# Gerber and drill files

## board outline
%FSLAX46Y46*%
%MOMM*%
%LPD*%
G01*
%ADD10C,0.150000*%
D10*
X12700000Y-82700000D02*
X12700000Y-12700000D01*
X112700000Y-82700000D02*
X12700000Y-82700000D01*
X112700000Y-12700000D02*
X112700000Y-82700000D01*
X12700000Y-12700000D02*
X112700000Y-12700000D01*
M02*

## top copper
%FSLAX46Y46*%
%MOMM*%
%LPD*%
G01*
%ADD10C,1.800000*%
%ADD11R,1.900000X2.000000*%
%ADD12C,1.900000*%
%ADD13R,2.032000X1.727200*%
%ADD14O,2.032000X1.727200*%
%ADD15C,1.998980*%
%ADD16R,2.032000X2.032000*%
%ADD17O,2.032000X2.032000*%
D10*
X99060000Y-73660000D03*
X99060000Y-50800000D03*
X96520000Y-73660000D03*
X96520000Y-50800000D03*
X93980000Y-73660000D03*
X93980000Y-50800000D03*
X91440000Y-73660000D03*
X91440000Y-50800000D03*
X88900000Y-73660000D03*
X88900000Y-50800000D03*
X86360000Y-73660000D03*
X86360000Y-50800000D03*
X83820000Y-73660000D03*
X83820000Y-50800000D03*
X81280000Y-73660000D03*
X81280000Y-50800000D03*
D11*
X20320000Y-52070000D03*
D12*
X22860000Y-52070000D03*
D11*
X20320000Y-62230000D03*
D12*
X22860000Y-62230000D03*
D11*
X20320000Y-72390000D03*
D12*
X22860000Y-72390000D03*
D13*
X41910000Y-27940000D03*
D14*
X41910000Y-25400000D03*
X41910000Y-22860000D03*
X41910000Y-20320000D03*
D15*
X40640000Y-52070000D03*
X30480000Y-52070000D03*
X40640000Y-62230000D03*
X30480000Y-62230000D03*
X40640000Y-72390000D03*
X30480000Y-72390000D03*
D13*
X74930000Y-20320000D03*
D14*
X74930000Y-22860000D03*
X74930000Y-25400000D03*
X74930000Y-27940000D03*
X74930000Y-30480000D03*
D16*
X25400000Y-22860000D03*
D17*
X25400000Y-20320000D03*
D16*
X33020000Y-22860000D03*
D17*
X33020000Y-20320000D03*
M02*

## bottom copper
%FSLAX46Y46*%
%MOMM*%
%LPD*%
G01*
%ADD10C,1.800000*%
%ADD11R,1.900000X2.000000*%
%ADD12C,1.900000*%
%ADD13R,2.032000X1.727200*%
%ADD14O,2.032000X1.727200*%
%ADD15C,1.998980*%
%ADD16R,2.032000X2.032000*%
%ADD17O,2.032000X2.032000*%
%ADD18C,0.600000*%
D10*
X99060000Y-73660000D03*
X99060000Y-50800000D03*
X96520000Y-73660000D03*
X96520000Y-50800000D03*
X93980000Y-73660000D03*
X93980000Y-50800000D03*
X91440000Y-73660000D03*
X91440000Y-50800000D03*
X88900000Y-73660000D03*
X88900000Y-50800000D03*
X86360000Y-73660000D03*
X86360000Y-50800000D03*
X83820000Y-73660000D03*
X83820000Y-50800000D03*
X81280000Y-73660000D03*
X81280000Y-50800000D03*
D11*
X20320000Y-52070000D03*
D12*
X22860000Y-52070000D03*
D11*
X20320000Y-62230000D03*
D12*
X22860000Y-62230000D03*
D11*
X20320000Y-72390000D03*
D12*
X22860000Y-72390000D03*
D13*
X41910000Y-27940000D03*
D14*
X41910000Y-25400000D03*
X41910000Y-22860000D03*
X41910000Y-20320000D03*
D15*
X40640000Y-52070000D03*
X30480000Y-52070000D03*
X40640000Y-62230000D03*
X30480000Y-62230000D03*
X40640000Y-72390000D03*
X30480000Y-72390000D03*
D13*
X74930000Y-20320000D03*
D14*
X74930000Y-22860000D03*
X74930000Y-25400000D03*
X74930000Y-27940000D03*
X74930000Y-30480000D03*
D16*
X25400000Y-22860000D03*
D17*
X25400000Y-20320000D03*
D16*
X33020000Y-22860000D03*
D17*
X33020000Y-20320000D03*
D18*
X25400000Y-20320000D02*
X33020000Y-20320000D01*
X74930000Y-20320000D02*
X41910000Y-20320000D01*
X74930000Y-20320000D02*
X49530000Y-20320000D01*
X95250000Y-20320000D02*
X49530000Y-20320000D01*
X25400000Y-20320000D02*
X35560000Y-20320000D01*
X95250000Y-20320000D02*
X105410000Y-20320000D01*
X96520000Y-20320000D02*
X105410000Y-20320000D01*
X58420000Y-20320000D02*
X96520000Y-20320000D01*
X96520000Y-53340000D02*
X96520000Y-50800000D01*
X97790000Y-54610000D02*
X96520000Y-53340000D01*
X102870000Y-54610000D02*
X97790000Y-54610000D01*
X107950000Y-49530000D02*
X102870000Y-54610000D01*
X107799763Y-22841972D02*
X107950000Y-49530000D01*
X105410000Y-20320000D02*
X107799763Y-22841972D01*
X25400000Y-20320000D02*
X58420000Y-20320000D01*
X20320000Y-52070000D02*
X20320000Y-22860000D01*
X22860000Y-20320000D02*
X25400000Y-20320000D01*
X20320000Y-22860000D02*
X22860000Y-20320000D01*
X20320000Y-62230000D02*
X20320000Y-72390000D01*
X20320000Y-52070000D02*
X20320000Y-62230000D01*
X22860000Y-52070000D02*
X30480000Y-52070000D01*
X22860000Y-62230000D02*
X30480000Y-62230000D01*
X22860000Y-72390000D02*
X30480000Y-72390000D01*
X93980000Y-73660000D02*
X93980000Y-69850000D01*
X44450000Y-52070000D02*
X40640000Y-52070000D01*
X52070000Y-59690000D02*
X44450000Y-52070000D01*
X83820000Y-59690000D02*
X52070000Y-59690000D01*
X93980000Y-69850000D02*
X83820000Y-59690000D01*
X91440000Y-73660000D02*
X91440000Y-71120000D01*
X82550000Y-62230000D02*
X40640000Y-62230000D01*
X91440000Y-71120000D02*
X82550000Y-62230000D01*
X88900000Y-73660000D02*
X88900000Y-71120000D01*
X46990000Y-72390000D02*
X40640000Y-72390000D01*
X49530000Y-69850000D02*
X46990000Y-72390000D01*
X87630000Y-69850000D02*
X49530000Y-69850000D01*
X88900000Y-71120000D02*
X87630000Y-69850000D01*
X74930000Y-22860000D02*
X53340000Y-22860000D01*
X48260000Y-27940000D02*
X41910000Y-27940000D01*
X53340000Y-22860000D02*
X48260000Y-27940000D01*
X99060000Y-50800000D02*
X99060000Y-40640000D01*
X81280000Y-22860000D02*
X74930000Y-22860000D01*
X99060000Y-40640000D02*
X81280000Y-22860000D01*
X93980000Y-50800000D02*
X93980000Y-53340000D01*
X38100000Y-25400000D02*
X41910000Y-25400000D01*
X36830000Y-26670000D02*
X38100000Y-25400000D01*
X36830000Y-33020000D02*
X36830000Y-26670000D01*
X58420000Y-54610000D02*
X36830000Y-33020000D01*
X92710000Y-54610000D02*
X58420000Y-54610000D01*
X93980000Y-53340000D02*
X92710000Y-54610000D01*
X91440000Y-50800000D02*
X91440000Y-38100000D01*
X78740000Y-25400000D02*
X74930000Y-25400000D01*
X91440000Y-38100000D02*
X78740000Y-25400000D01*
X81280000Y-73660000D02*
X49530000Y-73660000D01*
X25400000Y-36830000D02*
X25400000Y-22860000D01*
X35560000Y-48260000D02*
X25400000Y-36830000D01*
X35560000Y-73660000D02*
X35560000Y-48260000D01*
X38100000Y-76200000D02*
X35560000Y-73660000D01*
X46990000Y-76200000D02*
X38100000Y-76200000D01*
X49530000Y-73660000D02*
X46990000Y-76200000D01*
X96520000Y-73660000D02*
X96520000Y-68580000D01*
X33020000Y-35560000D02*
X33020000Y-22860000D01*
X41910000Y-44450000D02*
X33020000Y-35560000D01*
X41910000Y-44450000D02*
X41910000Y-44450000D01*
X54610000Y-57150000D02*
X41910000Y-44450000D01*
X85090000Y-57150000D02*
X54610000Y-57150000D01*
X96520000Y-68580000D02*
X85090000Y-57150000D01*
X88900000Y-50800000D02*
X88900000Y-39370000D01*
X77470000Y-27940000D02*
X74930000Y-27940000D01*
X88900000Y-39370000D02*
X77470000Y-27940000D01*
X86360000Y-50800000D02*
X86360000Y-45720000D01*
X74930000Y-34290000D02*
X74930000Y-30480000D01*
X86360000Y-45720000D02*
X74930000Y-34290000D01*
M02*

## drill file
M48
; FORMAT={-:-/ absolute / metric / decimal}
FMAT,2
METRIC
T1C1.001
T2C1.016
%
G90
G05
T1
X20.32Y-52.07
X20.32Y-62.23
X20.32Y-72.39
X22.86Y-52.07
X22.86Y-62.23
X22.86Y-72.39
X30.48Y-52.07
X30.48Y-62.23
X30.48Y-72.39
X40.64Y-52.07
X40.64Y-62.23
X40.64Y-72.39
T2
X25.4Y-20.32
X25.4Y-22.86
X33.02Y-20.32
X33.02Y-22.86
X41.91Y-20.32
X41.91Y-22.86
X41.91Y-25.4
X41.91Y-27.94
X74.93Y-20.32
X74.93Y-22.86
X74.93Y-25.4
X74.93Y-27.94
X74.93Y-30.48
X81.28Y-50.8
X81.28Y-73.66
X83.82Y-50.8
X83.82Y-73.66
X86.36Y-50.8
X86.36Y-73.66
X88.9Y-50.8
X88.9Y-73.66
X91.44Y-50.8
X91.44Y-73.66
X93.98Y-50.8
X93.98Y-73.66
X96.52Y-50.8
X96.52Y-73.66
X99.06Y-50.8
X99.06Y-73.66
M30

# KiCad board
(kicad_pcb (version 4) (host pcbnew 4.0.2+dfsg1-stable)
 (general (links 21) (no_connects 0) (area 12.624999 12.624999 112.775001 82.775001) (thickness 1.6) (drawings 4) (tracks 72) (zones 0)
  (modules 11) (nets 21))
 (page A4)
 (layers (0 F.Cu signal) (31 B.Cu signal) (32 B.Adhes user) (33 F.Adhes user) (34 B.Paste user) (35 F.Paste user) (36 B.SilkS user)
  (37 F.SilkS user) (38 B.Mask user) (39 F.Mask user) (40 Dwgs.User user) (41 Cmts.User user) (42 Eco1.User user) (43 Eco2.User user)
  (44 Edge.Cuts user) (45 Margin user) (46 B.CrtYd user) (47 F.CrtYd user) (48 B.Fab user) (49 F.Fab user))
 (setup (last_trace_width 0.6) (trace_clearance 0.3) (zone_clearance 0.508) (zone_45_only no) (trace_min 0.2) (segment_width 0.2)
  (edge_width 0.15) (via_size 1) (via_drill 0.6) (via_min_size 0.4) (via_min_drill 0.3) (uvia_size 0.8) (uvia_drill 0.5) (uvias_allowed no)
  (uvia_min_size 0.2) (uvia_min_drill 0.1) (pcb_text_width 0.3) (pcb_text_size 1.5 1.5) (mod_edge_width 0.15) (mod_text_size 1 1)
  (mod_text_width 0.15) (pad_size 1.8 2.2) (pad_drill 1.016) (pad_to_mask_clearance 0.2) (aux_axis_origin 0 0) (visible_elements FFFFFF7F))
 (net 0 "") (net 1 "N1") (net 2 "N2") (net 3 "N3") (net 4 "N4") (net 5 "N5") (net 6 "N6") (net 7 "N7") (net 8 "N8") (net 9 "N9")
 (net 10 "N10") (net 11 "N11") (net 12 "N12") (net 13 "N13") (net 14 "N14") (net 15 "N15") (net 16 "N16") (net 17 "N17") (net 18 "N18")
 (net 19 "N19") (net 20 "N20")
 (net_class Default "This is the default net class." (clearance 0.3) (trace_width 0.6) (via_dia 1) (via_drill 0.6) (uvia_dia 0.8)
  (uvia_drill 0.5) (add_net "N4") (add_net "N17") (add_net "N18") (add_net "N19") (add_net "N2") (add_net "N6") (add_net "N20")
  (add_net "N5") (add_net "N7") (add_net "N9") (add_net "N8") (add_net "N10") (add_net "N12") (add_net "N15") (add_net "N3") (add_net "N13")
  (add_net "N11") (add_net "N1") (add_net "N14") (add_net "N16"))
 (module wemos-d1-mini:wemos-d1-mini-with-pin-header (layer F.Cu) (at 90.17 62.23 180)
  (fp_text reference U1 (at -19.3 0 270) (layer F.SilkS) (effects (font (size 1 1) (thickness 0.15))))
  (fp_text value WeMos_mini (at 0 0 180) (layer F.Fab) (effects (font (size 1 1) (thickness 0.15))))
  (pad 16 thru_hole circle (at -8.89 -11.43 180) (size 1.8 1.8) (drill 1.016) (layers *.Cu *.Mask) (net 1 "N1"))
  (pad 1 thru_hole circle (at -8.89 11.43 180) (size 1.8 1.8) (drill 1.016) (layers *.Cu *.Mask) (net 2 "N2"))
  (pad 15 thru_hole circle (at -6.35 -11.43 180) (size 1.8 1.8) (drill 1.016) (layers *.Cu *.Mask) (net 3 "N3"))
  (pad 2 thru_hole circle (at -6.35 11.43 180) (size 1.8 1.8) (drill 1.016) (layers *.Cu *.Mask) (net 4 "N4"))
  (pad 14 thru_hole circle (at -3.81 -11.43 180) (size 1.8 1.8) (drill 1.016) (layers *.Cu *.Mask) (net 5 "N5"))
  (pad 3 thru_hole circle (at -3.81 11.43 180) (size 1.8 1.8) (drill 1.016) (layers *.Cu *.Mask) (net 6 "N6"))
  (pad 13 thru_hole circle (at -1.27 -11.43 180) (size 1.8 1.8) (drill 1.016) (layers *.Cu *.Mask) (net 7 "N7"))
  (pad 4 thru_hole circle (at -1.27 11.43 180) (size 1.8 1.8) (drill 1.016) (layers *.Cu *.Mask) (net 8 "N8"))
  (pad 12 thru_hole circle (at 1.27 -11.43 180) (size 1.8 1.8) (drill 1.016) (layers *.Cu *.Mask) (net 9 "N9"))
  (pad 5 thru_hole circle (at 1.27 11.43 180) (size 1.8 1.8) (drill 1.016) (layers *.Cu *.Mask) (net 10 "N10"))
  (pad 11 thru_hole circle (at 3.81 -11.43 180) (size 1.8 1.8) (drill 1.016) (layers *.Cu *.Mask) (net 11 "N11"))
  (pad 6 thru_hole circle (at 3.81 11.43 180) (size 1.8 1.8) (drill 1.016) (layers *.Cu *.Mask) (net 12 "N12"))
  (pad 10 thru_hole circle (at 6.35 -11.43 180) (size 1.8 1.8) (drill 1.016) (layers *.Cu *.Mask) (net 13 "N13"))
  (pad 7 thru_hole circle (at 6.35 11.43 180) (size 1.8 1.8) (drill 1.016) (layers *.Cu *.Mask) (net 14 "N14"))
  (pad 9 thru_hole circle (at 8.89 -11.43 180) (size 1.8 1.8) (drill 1.016) (layers *.Cu *.Mask) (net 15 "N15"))
  (pad 8 thru_hole circle (at 8.89 11.43 180) (size 1.8 1.8) (drill 1.016) (layers *.Cu *.Mask) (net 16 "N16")))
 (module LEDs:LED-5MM (layer F.Cu) (at 20.32 52.07)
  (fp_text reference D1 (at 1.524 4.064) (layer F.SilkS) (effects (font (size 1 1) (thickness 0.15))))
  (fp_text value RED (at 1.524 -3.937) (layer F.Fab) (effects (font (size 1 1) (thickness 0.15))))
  (pad 1 thru_hole rect (at 0 0 90) (size 2 1.9) (drill 1.00076) (layers *.Cu *.Mask F.SilkS) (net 4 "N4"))
  (pad 2 thru_hole circle (at 2.54 0) (size 1.9 1.9) (drill 1.00076) (layers *.Cu *.Mask F.SilkS) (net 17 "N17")))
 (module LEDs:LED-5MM (layer F.Cu) (at 20.32 62.23)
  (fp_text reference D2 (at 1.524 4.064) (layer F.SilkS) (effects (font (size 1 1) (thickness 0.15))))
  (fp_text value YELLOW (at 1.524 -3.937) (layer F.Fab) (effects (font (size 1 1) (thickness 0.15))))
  (pad 1 thru_hole rect (at 0 0 90) (size 2 1.9) (drill 1.00076) (layers *.Cu *.Mask F.SilkS) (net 4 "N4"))
  (pad 2 thru_hole circle (at 2.54 0) (size 1.9 1.9) (drill 1.00076) (layers *.Cu *.Mask F.SilkS) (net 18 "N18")))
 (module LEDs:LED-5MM (layer F.Cu) (at 20.32 72.39)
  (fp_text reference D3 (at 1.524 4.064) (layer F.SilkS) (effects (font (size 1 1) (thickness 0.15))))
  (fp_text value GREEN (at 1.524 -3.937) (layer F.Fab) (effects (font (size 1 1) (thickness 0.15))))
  (pad 1 thru_hole rect (at 0 0 90) (size 2 1.9) (drill 1.00076) (layers *.Cu *.Mask F.SilkS) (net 4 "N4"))
  (pad 2 thru_hole circle (at 2.54 0) (size 1.9 1.9) (drill 1.00076) (layers *.Cu *.Mask F.SilkS) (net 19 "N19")))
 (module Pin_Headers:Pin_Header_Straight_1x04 (layer F.Cu) (at 41.91 27.94 180)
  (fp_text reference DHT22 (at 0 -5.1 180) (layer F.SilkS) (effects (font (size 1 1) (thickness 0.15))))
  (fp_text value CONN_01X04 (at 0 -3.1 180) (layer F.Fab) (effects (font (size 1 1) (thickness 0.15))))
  (pad 1 thru_hole rect (at 0 0 180) (size 2.032 1.7272) (drill 1.016) (layers *.Cu *.Mask F.SilkS) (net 2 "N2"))
  (pad 2 thru_hole oval (at 0 2.54 180) (size 2.032 1.7272) (drill 1.016) (layers *.Cu *.Mask F.SilkS) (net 6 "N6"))
  (pad 3 thru_hole oval (at 0 5.08 180) (size 2.032 1.7272) (drill 1.016) (layers *.Cu *.Mask F.SilkS) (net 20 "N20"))
  (pad 4 thru_hole oval (at 0 7.62 180) (size 2.032 1.7272) (drill 1.016) (layers *.Cu *.Mask F.SilkS) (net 4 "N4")))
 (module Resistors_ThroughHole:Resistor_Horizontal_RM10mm (layer F.Cu) (at 40.64 52.07 180)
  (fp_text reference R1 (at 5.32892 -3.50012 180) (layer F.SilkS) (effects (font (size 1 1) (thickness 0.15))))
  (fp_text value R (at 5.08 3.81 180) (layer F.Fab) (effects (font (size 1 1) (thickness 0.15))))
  (pad 1 thru_hole circle (at 0 0 180) (size 1.99898 1.99898) (drill 1.00076) (layers *.Cu *.SilkS *.Mask) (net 5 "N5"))
  (pad 2 thru_hole circle (at 10.16 0 180) (size 1.99898 1.99898) (drill 1.00076) (layers *.Cu *.SilkS *.Mask) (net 17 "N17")))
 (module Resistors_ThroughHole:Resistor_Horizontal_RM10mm (layer F.Cu) (at 40.64 62.23 180)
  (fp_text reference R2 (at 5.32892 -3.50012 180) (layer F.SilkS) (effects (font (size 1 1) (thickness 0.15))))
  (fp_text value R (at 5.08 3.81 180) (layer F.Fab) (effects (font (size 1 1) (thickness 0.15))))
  (pad 1 thru_hole circle (at 0 0 180) (size 1.99898 1.99898) (drill 1.00076) (layers *.Cu *.SilkS *.Mask) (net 7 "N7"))
  (pad 2 thru_hole circle (at 10.16 0 180) (size 1.99898 1.99898) (drill 1.00076) (layers *.Cu *.SilkS *.Mask) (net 18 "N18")))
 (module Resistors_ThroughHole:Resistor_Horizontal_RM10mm (layer F.Cu) (at 40.64 72.39 180)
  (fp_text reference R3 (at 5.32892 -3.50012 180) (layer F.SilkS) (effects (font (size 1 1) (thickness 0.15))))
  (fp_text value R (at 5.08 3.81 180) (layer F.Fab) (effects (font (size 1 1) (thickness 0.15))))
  (pad 1 thru_hole circle (at 0 0 180) (size 1.99898 1.99898) (drill 1.00076) (layers *.Cu *.SilkS *.Mask) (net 9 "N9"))
  (pad 2 thru_hole circle (at 10.16 0 180) (size 1.99898 1.99898) (drill 1.00076) (layers *.Cu *.SilkS *.Mask) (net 19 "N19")))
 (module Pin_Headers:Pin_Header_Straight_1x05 (layer F.Cu) (at 74.93 20.32)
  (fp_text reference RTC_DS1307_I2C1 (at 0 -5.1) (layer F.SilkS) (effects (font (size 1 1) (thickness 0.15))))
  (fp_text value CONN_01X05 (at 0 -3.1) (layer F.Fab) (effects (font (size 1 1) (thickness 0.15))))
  (pad 1 thru_hole rect (at 0 0) (size 2.032 1.7272) (drill 1.016) (layers *.Cu *.Mask F.SilkS) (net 4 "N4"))
  (pad 2 thru_hole oval (at 0 2.54) (size 2.032 1.7272) (drill 1.016) (layers *.Cu *.Mask F.SilkS) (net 2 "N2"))
  (pad 3 thru_hole oval (at 0 5.08) (size 2.032 1.7272) (drill 1.016) (layers *.Cu *.Mask F.SilkS) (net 8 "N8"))
  (pad 4 thru_hole oval (at 0 7.62) (size 2.032 1.7272) (drill 1.016) (layers *.Cu *.Mask F.SilkS) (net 10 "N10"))
  (pad 5 thru_hole oval (at 0 10.16) (size 2.032 1.7272) (drill 1.016) (layers *.Cu *.Mask F.SilkS) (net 12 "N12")))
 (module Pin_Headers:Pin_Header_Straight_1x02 (layer F.Cu) (at 25.4 22.86 180)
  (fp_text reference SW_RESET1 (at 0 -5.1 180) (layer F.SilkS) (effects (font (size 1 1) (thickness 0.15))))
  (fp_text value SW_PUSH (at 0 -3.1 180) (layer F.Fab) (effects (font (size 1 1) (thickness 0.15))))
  (pad 1 thru_hole rect (at 0 0 180) (size 2.032 2.032) (drill 1.016) (layers *.Cu *.Mask F.SilkS) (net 15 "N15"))
  (pad 2 thru_hole oval (at 0 2.54 180) (size 2.032 2.032) (drill 1.016) (layers *.Cu *.Mask F.SilkS) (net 4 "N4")))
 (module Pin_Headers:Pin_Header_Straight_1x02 (layer F.Cu) (at 33.02 22.86 180)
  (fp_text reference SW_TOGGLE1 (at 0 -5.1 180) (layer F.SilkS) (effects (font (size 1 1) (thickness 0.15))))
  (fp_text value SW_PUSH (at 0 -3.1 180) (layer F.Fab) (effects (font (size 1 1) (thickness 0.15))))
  (pad 1 thru_hole rect (at 0 0 180) (size 2.032 2.032) (drill 1.016) (layers *.Cu *.Mask F.SilkS) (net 3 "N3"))
  (pad 2 thru_hole oval (at 0 2.54 180) (size 2.032 2.032) (drill 1.016) (layers *.Cu *.Mask F.SilkS) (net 4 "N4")))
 (gr_line (start 12.7 82.7) (end 12.7 12.7) (angle 90) (layer Edge.Cuts) (width 0.15))
 (gr_line (start 112.7 82.7) (end 12.7 82.7) (angle 90) (layer Edge.Cuts) (width 0.15))
 (gr_line (start 112.7 12.7) (end 112.7 82.7) (angle 90) (layer Edge.Cuts) (width 0.15))
 (gr_line (start 12.7 12.7) (end 112.7 12.7) (angle 90) (layer Edge.Cuts) (width 0.15))
 (segment (start 25.4 20.32) (end 33.02 20.32) (width 0.6) (layer B.Cu) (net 4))
 (segment (start 74.93 20.32) (end 41.91 20.32) (width 0.6) (layer B.Cu) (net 4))
 (segment (start 74.93 20.32) (end 49.53 20.32) (width 0.6) (layer B.Cu) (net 4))
 (segment (start 95.25 20.32) (end 49.53 20.32) (width 0.6) (layer B.Cu) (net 4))
 (segment (start 25.4 20.32) (end 35.56 20.32) (width 0.6) (layer B.Cu) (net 4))
 (segment (start 95.25 20.32) (end 105.41 20.32) (width 0.6) (layer B.Cu) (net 4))
 (segment (start 96.52 20.32) (end 105.41 20.32) (width 0.6) (layer B.Cu) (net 4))
 (segment (start 58.42 20.32) (end 96.52 20.32) (width 0.6) (layer B.Cu) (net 4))
 (segment (start 96.52 53.34) (end 96.52 50.8) (width 0.6) (layer B.Cu) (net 4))
 (segment (start 97.79 54.61) (end 96.52 53.34) (width 0.6) (layer B.Cu) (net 4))
 (segment (start 102.87 54.61) (end 97.79 54.61) (width 0.6) (layer B.Cu) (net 4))
 (segment (start 107.95 49.53) (end 102.87 54.61) (width 0.6) (layer B.Cu) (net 4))
 (segment (start 107.799763 22.841972) (end 107.95 49.53) (width 0.6) (layer B.Cu) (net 4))
 (segment (start 105.41 20.32) (end 107.799763 22.841972) (width 0.6) (layer B.Cu) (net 4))
 (segment (start 25.4 20.32) (end 58.42 20.32) (width 0.6) (layer B.Cu) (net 4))
 (segment (start 20.32 52.07) (end 20.32 22.86) (width 0.6) (layer B.Cu) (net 4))
 (segment (start 22.86 20.32) (end 25.4 20.32) (width 0.6) (layer B.Cu) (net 4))
 (segment (start 20.32 22.86) (end 22.86 20.32) (width 0.6) (layer B.Cu) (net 4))
 (segment (start 20.32 62.23) (end 20.32 72.39) (width 0.6) (layer B.Cu) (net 4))
 (segment (start 20.32 52.07) (end 20.32 62.23) (width 0.6) (layer B.Cu) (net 4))
 (segment (start 22.86 52.07) (end 30.48 52.07) (width 0.6) (layer B.Cu) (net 17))
 (segment (start 22.86 62.23) (end 30.48 62.23) (width 0.6) (layer B.Cu) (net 18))
 (segment (start 22.86 72.39) (end 30.48 72.39) (width 0.6) (layer B.Cu) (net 19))
 (segment (start 93.98 73.66) (end 93.98 69.85) (width 0.6) (layer B.Cu) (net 5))
 (segment (start 44.45 52.07) (end 40.64 52.07) (width 0.6) (layer B.Cu) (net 5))
 (segment (start 52.07 59.69) (end 44.45 52.07) (width 0.6) (layer B.Cu) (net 5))
 (segment (start 83.82 59.69) (end 52.07 59.69) (width 0.6) (layer B.Cu) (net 5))
 (segment (start 93.98 69.85) (end 83.82 59.69) (width 0.6) (layer B.Cu) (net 5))
 (segment (start 91.44 73.66) (end 91.44 71.12) (width 0.6) (layer B.Cu) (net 7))
 (segment (start 82.55 62.23) (end 40.64 62.23) (width 0.6) (layer B.Cu) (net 7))
 (segment (start 91.44 71.12) (end 82.55 62.23) (width 0.6) (layer B.Cu) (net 7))
 (segment (start 88.9 73.66) (end 88.9 71.12) (width 0.6) (layer B.Cu) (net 9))
 (segment (start 46.99 72.39) (end 40.64 72.39) (width 0.6) (layer B.Cu) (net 9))
 (segment (start 49.53 69.85) (end 46.99 72.39) (width 0.6) (layer B.Cu) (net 9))
 (segment (start 87.63 69.85) (end 49.53 69.85) (width 0.6) (layer B.Cu) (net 9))
 (segment (start 88.9 71.12) (end 87.63 69.85) (width 0.6) (layer B.Cu) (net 9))
 (segment (start 74.93 22.86) (end 53.34 22.86) (width 0.6) (layer B.Cu) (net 2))
 (segment (start 48.26 27.94) (end 41.91 27.94) (width 0.6) (layer B.Cu) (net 2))
 (segment (start 53.34 22.86) (end 48.26 27.94) (width 0.6) (layer B.Cu) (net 2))
 (segment (start 99.06 50.8) (end 99.06 40.64) (width 0.6) (layer B.Cu) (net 2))
 (segment (start 81.28 22.86) (end 74.93 22.86) (width 0.6) (layer B.Cu) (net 2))
 (segment (start 99.06 40.64) (end 81.28 22.86) (width 0.6) (layer B.Cu) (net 2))
 (segment (start 93.98 50.8) (end 93.98 53.34) (width 0.6) (layer B.Cu) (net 6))
 (segment (start 38.1 25.4) (end 41.91 25.4) (width 0.6) (layer B.Cu) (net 6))
 (segment (start 36.83 26.67) (end 38.1 25.4) (width 0.6) (layer B.Cu) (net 6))
 (segment (start 36.83 33.02) (end 36.83 26.67) (width 0.6) (layer B.Cu) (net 6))
 (segment (start 58.42 54.61) (end 36.83 33.02) (width 0.6) (layer B.Cu) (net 6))
 (segment (start 92.71 54.61) (end 58.42 54.61) (width 0.6) (layer B.Cu) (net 6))
 (segment (start 93.98 53.34) (end 92.71 54.61) (width 0.6) (layer B.Cu) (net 6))
 (segment (start 91.44 50.8) (end 91.44 38.1) (width 0.6) (layer B.Cu) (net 8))
 (segment (start 78.74 25.4) (end 74.93 25.4) (width 0.6) (layer B.Cu) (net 8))
 (segment (start 91.44 38.1) (end 78.74 25.4) (width 0.6) (layer B.Cu) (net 8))
 (segment (start 81.28 73.66) (end 49.53 73.66) (width 0.6) (layer B.Cu) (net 15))
 (segment (start 25.4 36.83) (end 25.4 22.86) (width 0.6) (layer B.Cu) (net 15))
 (segment (start 35.56 48.26) (end 25.4 36.83) (width 0.6) (layer B.Cu) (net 15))
 (segment (start 35.56 73.66) (end 35.56 48.26) (width 0.6) (layer B.Cu) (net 15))
 (segment (start 38.1 76.2) (end 35.56 73.66) (width 0.6) (layer B.Cu) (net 15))
 (segment (start 46.99 76.2) (end 38.1 76.2) (width 0.6) (layer B.Cu) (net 15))
 (segment (start 49.53 73.66) (end 46.99 76.2) (width 0.6) (layer B.Cu) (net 15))
 (segment (start 96.52 73.66) (end 96.52 68.58) (width 0.6) (layer B.Cu) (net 3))
 (segment (start 33.02 35.56) (end 33.02 22.86) (width 0.6) (layer B.Cu) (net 3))
 (segment (start 41.91 44.45) (end 33.02 35.56) (width 0.6) (layer B.Cu) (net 3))
 (segment (start 41.91 44.45) (end 41.91 44.45) (width 0.6) (layer B.Cu) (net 3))
 (segment (start 54.61 57.15) (end 41.91 44.45) (width 0.6) (layer B.Cu) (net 3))
 (segment (start 85.09 57.15) (end 54.61 57.15) (width 0.6) (layer B.Cu) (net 3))
 (segment (start 96.52 68.58) (end 85.09 57.15) (width 0.6) (layer B.Cu) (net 3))
 (segment (start 88.9 50.8) (end 88.9 39.37) (width 0.6) (layer B.Cu) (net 10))
 (segment (start 77.47 27.94) (end 74.93 27.94) (width 0.6) (layer B.Cu) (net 10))
 (segment (start 88.9 39.37) (end 77.47 27.94) (width 0.6) (layer B.Cu) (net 10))
 (segment (start 86.36 50.8) (end 86.36 45.72) (width 0.6) (layer B.Cu) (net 12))
 (segment (start 74.93 34.29) (end 74.93 30.48) (width 0.6) (layer B.Cu) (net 12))
 (segment (start 86.36 45.72) (end 74.93 34.29) (width 0.6) (layer B.Cu) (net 12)))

